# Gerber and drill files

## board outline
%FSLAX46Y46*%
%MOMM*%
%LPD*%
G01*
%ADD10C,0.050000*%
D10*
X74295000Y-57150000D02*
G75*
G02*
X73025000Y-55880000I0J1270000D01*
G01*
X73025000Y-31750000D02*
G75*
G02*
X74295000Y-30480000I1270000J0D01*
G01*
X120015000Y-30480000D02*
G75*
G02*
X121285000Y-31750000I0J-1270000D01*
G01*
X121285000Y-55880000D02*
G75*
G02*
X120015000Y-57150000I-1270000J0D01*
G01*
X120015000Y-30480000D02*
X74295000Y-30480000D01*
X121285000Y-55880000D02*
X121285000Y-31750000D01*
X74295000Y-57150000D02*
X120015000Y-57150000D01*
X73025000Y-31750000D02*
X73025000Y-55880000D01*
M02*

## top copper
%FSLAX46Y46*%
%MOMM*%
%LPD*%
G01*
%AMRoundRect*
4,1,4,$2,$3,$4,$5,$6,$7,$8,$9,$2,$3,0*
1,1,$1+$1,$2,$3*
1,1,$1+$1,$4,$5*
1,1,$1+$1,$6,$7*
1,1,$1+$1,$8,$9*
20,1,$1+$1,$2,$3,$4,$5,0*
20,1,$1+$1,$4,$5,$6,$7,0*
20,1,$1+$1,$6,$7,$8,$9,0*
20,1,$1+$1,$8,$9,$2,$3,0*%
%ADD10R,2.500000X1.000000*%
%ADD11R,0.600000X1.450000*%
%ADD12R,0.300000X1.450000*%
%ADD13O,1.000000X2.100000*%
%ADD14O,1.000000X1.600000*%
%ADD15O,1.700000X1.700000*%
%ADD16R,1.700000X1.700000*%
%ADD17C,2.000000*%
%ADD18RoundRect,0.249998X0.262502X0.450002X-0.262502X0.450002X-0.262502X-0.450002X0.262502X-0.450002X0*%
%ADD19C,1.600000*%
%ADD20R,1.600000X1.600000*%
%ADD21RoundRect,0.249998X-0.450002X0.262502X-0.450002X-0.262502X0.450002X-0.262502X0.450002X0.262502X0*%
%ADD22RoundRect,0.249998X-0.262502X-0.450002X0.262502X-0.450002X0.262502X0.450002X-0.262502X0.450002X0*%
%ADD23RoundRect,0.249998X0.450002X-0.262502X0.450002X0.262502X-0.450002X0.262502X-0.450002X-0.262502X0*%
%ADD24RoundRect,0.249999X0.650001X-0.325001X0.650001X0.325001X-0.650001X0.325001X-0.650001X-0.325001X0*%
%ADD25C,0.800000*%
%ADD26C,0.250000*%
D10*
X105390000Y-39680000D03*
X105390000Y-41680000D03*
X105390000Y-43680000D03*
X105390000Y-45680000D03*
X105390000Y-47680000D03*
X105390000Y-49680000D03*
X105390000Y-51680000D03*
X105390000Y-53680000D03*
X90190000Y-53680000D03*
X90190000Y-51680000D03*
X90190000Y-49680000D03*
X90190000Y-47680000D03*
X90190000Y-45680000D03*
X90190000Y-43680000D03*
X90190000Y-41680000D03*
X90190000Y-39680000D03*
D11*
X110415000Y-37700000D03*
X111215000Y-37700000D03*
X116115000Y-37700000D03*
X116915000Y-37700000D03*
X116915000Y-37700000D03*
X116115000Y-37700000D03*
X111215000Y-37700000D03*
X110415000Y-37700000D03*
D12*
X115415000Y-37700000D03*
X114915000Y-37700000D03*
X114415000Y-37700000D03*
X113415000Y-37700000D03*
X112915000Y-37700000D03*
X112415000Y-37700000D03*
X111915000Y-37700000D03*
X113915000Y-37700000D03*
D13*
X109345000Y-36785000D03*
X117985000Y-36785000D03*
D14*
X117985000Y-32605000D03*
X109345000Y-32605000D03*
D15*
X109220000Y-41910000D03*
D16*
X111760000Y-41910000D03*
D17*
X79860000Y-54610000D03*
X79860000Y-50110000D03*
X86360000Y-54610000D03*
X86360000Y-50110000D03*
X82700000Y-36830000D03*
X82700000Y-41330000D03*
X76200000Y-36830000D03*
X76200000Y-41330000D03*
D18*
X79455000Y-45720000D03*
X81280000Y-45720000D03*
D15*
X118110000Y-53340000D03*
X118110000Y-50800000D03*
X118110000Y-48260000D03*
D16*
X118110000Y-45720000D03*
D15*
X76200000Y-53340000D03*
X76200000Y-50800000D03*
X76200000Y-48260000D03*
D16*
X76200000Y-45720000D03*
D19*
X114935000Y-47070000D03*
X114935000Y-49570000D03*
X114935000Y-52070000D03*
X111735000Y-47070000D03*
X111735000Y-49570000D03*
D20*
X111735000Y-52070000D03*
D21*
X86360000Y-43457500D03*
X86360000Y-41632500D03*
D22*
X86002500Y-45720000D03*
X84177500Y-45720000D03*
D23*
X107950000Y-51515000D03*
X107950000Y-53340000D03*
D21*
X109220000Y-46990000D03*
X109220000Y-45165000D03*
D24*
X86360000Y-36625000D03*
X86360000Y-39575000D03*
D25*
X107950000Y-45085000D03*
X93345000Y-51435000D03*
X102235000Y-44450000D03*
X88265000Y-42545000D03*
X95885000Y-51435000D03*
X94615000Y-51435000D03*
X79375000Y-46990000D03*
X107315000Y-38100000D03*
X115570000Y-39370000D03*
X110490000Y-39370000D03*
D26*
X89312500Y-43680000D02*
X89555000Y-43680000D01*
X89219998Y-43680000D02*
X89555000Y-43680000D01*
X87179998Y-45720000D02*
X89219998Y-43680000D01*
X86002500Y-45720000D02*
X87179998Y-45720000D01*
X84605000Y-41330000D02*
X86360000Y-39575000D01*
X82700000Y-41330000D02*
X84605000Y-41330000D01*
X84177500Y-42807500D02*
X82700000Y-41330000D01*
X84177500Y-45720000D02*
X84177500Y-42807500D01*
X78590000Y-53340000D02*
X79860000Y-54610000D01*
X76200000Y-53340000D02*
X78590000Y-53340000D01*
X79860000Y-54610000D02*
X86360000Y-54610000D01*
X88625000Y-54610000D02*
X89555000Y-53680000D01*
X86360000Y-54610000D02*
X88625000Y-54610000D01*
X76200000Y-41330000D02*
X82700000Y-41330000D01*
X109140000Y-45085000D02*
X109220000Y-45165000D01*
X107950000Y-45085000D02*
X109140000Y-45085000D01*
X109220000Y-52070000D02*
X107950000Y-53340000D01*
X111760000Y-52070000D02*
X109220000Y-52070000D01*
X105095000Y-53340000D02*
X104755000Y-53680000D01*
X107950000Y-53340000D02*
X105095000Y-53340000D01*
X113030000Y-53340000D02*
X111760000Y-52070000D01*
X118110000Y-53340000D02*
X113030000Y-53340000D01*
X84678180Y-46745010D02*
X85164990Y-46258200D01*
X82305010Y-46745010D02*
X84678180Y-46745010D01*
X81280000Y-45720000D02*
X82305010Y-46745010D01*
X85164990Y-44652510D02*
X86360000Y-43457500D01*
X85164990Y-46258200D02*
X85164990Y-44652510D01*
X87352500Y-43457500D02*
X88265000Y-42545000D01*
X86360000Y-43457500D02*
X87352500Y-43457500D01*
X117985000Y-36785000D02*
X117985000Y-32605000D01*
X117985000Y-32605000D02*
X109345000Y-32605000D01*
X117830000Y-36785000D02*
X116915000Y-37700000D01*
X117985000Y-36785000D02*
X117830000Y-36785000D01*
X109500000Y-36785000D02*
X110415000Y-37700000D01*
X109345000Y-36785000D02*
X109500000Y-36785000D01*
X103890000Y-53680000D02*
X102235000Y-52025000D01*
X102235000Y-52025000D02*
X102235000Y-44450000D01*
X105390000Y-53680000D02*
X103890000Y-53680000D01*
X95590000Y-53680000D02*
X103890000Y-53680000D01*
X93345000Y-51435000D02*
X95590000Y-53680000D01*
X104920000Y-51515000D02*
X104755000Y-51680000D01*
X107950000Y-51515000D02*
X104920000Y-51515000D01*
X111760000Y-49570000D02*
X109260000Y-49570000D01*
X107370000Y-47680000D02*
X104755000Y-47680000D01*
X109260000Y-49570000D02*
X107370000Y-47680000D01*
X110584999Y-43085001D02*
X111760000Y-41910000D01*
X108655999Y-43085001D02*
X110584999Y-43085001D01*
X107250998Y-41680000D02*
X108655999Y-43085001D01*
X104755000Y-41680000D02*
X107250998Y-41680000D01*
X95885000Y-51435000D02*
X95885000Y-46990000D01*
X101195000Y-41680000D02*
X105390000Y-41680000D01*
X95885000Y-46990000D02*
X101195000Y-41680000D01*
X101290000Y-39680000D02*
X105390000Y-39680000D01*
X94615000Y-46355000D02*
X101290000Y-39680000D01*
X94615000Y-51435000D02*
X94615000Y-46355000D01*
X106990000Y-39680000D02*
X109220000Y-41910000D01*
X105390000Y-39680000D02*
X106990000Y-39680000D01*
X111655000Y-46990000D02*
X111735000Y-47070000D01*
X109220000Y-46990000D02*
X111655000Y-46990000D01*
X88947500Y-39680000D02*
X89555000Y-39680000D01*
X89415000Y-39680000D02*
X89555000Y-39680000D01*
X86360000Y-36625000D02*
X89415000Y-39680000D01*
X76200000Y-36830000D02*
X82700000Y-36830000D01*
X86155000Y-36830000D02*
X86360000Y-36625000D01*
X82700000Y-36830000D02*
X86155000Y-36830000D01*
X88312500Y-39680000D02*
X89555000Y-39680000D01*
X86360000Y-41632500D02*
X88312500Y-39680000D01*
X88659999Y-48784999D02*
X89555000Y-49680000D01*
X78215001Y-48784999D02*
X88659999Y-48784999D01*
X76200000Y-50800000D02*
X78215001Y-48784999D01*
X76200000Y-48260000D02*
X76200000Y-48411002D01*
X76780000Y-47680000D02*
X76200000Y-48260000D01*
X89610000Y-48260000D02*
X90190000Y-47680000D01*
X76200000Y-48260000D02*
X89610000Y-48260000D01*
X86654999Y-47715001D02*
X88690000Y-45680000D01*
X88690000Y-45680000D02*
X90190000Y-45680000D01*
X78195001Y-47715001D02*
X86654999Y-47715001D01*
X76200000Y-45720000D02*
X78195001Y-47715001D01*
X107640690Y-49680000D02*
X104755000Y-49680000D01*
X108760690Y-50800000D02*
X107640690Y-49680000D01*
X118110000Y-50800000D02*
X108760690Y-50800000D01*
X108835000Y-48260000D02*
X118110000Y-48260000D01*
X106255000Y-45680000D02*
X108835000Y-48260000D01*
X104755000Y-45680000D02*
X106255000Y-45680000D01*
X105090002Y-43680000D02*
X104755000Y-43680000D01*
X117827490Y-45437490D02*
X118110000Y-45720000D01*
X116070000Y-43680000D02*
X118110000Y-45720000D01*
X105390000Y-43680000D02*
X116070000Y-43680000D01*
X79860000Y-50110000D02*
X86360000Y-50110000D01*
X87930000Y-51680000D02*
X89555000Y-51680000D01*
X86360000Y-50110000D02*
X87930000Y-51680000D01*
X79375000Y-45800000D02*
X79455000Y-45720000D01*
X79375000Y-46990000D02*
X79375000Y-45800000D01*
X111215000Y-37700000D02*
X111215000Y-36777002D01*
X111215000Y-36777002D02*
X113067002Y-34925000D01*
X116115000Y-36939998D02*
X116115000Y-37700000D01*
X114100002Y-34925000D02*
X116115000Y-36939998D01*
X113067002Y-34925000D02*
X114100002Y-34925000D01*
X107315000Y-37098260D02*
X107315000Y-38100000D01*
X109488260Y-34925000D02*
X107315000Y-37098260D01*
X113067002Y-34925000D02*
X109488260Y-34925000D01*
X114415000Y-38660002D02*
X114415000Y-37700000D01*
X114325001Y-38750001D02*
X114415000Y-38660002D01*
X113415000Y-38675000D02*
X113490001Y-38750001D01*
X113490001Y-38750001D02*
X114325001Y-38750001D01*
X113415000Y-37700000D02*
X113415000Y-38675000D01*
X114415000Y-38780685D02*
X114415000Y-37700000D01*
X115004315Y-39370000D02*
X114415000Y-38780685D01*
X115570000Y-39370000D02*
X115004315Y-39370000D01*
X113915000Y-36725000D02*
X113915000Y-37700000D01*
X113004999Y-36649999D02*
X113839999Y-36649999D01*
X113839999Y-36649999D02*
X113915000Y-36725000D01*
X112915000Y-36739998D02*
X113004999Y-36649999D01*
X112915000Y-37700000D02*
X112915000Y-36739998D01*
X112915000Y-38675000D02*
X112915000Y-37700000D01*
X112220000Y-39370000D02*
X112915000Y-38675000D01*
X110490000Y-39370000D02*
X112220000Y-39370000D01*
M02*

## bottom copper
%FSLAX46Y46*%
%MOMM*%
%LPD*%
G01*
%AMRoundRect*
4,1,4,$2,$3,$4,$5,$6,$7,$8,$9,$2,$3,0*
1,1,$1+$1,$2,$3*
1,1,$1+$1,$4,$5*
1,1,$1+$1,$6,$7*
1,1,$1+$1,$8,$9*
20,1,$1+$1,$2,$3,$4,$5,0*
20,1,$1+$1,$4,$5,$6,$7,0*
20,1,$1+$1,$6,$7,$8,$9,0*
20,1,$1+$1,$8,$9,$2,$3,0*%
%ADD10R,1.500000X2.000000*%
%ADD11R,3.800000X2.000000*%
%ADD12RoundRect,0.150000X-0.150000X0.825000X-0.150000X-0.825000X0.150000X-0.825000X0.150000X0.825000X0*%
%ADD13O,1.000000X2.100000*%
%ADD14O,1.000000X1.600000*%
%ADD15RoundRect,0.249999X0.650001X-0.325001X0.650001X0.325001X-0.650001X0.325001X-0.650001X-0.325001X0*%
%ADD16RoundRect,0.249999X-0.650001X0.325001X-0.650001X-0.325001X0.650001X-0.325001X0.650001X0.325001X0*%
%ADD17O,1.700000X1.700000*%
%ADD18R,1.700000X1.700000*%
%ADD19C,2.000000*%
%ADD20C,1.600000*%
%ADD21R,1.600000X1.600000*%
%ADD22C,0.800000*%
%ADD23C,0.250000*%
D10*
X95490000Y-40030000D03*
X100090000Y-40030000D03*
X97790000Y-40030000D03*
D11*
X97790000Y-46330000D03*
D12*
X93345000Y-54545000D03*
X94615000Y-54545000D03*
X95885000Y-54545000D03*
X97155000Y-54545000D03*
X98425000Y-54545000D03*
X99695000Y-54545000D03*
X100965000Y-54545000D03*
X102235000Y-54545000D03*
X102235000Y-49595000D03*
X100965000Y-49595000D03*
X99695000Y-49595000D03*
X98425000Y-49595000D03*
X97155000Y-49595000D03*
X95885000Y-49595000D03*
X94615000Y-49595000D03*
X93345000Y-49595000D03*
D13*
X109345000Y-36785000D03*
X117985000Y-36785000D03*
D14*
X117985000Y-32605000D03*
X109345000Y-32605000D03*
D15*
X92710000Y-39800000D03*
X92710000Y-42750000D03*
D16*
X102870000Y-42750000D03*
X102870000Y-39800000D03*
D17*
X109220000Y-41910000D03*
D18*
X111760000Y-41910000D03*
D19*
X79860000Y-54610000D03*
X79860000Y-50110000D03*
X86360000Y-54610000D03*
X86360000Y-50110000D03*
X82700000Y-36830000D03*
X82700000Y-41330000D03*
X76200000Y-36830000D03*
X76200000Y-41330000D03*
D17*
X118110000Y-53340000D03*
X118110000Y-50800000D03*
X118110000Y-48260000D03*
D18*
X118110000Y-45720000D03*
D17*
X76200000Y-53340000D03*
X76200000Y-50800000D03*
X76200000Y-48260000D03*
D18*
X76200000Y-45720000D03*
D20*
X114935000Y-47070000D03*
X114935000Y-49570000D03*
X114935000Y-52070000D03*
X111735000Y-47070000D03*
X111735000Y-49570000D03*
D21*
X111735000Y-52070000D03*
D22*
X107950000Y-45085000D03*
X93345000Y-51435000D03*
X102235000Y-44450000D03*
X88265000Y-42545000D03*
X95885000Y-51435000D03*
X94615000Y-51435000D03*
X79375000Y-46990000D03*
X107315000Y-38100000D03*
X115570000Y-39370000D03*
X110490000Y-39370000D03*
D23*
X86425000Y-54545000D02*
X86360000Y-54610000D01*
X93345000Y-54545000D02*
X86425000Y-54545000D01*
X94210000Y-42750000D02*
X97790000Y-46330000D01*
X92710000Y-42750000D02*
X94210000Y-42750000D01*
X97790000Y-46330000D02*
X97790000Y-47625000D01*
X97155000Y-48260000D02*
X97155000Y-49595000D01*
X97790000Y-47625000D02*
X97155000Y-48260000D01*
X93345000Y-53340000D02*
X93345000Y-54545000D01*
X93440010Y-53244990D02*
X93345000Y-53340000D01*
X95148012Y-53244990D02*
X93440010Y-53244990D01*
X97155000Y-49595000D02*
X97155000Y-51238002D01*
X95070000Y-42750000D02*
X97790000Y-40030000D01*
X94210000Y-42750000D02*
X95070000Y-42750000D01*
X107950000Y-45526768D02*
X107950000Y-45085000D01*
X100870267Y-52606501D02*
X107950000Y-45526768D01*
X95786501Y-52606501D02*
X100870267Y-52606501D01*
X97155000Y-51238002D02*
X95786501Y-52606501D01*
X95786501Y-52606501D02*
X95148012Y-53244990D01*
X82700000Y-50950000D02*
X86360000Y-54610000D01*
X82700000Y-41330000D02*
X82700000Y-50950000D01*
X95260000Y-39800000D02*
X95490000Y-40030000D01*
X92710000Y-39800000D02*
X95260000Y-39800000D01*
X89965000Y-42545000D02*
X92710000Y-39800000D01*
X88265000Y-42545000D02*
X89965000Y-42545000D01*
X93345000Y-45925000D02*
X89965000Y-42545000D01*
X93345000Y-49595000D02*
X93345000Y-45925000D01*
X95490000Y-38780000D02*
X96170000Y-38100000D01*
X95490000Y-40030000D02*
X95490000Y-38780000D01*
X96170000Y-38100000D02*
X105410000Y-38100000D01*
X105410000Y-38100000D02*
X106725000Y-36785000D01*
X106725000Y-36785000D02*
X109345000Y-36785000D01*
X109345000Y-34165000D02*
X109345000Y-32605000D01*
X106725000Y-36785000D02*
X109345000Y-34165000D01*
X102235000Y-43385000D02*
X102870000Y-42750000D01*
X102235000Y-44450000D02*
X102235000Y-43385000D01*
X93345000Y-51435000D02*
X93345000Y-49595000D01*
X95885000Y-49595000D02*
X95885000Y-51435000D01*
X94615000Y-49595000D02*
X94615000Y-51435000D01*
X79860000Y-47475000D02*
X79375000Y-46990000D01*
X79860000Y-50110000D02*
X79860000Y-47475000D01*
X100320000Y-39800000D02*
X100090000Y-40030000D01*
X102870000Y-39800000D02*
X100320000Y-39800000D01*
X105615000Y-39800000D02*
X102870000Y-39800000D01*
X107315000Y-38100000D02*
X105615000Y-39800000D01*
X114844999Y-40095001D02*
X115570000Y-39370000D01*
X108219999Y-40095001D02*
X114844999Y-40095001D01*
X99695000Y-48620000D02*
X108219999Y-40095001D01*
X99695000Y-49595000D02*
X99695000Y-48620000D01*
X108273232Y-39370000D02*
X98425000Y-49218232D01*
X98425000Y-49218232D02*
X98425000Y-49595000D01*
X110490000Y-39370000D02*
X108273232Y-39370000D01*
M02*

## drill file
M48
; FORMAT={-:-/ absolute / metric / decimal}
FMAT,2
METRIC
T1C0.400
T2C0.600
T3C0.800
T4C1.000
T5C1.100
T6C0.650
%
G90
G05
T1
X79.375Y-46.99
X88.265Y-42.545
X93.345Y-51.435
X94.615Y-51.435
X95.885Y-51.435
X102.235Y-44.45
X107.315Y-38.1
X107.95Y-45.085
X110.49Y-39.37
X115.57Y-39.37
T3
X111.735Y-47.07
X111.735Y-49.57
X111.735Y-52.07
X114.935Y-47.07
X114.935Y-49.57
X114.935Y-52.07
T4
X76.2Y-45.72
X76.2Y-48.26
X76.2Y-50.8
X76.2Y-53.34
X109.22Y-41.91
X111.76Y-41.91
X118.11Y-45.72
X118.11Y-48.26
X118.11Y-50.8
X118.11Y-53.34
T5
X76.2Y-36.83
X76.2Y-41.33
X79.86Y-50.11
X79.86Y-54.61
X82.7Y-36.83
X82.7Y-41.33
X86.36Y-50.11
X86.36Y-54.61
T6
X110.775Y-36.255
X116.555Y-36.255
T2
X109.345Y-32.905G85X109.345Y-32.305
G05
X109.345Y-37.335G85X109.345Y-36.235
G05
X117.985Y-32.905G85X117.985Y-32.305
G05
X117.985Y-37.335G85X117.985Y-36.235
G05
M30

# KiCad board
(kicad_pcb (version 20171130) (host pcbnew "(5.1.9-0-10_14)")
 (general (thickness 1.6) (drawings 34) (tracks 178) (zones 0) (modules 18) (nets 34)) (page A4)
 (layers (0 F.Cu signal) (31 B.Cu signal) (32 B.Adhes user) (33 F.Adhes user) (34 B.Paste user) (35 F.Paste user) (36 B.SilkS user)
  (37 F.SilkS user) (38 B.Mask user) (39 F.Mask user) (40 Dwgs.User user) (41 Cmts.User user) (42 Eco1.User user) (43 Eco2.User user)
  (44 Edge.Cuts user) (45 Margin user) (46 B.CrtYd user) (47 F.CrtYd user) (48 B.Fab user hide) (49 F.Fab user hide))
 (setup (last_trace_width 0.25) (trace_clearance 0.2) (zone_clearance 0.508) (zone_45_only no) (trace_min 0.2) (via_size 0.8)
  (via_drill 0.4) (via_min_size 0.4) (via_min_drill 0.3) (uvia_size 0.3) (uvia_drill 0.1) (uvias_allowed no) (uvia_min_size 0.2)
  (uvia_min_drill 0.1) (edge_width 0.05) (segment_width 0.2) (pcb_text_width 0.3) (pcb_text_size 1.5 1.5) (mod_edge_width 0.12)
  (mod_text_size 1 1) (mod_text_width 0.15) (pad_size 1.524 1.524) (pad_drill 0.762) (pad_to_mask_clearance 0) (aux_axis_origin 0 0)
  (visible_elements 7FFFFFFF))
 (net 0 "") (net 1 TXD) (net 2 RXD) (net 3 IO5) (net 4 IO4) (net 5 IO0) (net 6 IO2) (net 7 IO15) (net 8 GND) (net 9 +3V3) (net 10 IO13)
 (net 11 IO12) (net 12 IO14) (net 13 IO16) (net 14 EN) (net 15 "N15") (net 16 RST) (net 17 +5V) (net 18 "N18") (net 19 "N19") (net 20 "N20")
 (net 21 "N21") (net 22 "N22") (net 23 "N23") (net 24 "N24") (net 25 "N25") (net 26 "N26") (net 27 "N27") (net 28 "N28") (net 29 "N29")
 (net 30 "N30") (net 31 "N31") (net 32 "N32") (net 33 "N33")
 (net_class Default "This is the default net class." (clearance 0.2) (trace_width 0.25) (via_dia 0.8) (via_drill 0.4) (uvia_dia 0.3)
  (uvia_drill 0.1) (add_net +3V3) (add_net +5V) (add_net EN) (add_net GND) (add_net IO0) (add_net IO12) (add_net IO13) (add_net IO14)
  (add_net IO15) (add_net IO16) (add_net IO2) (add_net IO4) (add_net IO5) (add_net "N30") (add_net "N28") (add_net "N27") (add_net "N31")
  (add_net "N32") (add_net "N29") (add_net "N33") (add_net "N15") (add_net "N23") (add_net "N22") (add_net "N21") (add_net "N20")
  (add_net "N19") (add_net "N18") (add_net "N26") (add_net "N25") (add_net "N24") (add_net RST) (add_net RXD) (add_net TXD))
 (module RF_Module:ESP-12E (layer F.Cu) (at 97.79 43.18)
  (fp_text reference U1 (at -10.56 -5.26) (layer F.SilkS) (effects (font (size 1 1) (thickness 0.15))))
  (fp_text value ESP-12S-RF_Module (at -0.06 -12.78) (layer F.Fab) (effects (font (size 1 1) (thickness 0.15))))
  (pad 16 smd rect (at 7.6 -3.5) (size 2.5 1) (layers F.Cu F.Paste F.Mask) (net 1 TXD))
  (pad 15 smd rect (at 7.6 -1.5) (size 2.5 1) (layers F.Cu F.Paste F.Mask) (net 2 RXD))
  (pad 14 smd rect (at 7.6 0.5) (size 2.5 1) (layers F.Cu F.Paste F.Mask) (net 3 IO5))
  (pad 13 smd rect (at 7.6 2.5) (size 2.5 1) (layers F.Cu F.Paste F.Mask) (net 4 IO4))
  (pad 12 smd rect (at 7.6 4.5) (size 2.5 1) (layers F.Cu F.Paste F.Mask) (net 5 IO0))
  (pad 11 smd rect (at 7.6 6.5) (size 2.5 1) (layers F.Cu F.Paste F.Mask) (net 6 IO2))
  (pad 10 smd rect (at 7.6 8.5) (size 2.5 1) (layers F.Cu F.Paste F.Mask) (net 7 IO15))
  (pad 9 smd rect (at 7.6 10.5) (size 2.5 1) (layers F.Cu F.Paste F.Mask) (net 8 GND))
  (pad 8 smd rect (at -7.6 10.5) (size 2.5 1) (layers F.Cu F.Paste F.Mask) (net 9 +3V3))
  (pad 7 smd rect (at -7.6 8.5) (size 2.5 1) (layers F.Cu F.Paste F.Mask) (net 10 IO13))
  (pad 6 smd rect (at -7.6 6.5) (size 2.5 1) (layers F.Cu F.Paste F.Mask) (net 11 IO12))
  (pad 5 smd rect (at -7.6 4.5) (size 2.5 1) (layers F.Cu F.Paste F.Mask) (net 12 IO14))
  (pad 4 smd rect (at -7.6 2.5) (size 2.5 1) (layers F.Cu F.Paste F.Mask) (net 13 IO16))
  (pad 3 smd rect (at -7.6 0.5) (size 2.5 1) (layers F.Cu F.Paste F.Mask) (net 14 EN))
  (pad 2 smd rect (at -7.6 -1.5) (size 2.5 1) (layers F.Cu F.Paste F.Mask) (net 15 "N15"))
  (pad 1 smd rect (at -7.6 -3.5) (size 2.5 1) (layers F.Cu F.Paste F.Mask) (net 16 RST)))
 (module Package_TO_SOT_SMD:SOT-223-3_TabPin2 (layer B.Cu) (at 97.79 43.18 270)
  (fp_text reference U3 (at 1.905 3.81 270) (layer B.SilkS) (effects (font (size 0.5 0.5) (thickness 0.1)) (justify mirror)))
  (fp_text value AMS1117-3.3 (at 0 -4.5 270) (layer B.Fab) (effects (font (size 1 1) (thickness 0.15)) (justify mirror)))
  (pad 1 smd rect (at -3.15 2.3 270) (size 2 1.5) (layers B.Cu B.Paste B.Mask) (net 8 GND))
  (pad 3 smd rect (at -3.15 -2.3 270) (size 2 1.5) (layers B.Cu B.Paste B.Mask) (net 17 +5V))
  (pad 2 smd rect (at -3.15 0 270) (size 2 1.5) (layers B.Cu B.Paste B.Mask) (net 9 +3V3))
  (pad 2 smd rect (at 3.15 0 270) (size 2 3.8) (layers B.Cu B.Paste B.Mask) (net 9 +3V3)))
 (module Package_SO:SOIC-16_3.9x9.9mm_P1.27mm (layer B.Cu) (at 97.79 52.07 270)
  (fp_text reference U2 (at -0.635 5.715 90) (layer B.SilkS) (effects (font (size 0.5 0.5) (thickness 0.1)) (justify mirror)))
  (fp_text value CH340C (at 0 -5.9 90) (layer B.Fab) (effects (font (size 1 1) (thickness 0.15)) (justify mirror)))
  (pad 16 smd roundrect (at 2.475 4.445 270) (size 1.95 0.6) (layers B.Cu B.Paste B.Mask) (roundrect_rratio 0.25) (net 9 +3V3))
  (pad 15 smd roundrect (at 2.475 3.175 270) (size 1.95 0.6) (layers B.Cu B.Paste B.Mask) (roundrect_rratio 0.25) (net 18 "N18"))
  (pad 14 smd roundrect (at 2.475 1.905 270) (size 1.95 0.6) (layers B.Cu B.Paste B.Mask) (roundrect_rratio 0.25) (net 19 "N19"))
  (pad 13 smd roundrect (at 2.475 0.635 270) (size 1.95 0.6) (layers B.Cu B.Paste B.Mask) (roundrect_rratio 0.25) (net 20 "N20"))
  (pad 12 smd roundrect (at 2.475 -0.635 270) (size 1.95 0.6) (layers B.Cu B.Paste B.Mask) (roundrect_rratio 0.25) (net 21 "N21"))
  (pad 11 smd roundrect (at 2.475 -1.905 270) (size 1.95 0.6) (layers B.Cu B.Paste B.Mask) (roundrect_rratio 0.25) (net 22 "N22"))
  (pad 10 smd roundrect (at 2.475 -3.175 270) (size 1.95 0.6) (layers B.Cu B.Paste B.Mask) (roundrect_rratio 0.25) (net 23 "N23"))
  (pad 9 smd roundrect (at 2.475 -4.445 270) (size 1.95 0.6) (layers B.Cu B.Paste B.Mask) (roundrect_rratio 0.25) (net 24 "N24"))
  (pad 8 smd roundrect (at -2.475 -4.445 270) (size 1.95 0.6) (layers B.Cu B.Paste B.Mask) (roundrect_rratio 0.25) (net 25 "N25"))
  (pad 7 smd roundrect (at -2.475 -3.175 270) (size 1.95 0.6) (layers B.Cu B.Paste B.Mask) (roundrect_rratio 0.25) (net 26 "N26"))
  (pad 6 smd roundrect (at -2.475 -1.905 270) (size 1.95 0.6) (layers B.Cu B.Paste B.Mask) (roundrect_rratio 0.25) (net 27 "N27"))
  (pad 5 smd roundrect (at -2.475 -0.635 270) (size 1.95 0.6) (layers B.Cu B.Paste B.Mask) (roundrect_rratio 0.25) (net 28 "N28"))
  (pad 4 smd roundrect (at -2.475 0.635 270) (size 1.95 0.6) (layers B.Cu B.Paste B.Mask) (roundrect_rratio 0.25) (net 9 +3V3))
  (pad 3 smd roundrect (at -2.475 1.905 270) (size 1.95 0.6) (layers B.Cu B.Paste B.Mask) (roundrect_rratio 0.25) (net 2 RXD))
  (pad 2 smd roundrect (at -2.475 3.175 270) (size 1.95 0.6) (layers B.Cu B.Paste B.Mask) (roundrect_rratio 0.25) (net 1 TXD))
  (pad 1 smd roundrect (at -2.475 4.445 270) (size 1.95 0.6) (layers B.Cu B.Paste B.Mask) (roundrect_rratio 0.25) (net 8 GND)))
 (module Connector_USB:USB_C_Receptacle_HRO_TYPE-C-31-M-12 (layer F.Cu) (at 113.665 33.655 180)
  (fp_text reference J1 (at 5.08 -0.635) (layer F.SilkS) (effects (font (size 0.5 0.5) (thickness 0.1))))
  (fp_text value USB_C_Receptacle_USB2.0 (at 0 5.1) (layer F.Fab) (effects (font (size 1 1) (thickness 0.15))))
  (pad B1 smd rect (at 3.25 -4.045 180) (size 0.6 1.45) (layers F.Cu F.Paste F.Mask) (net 8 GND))
  (pad A9 smd rect (at 2.45 -4.045 180) (size 0.6 1.45) (layers F.Cu F.Paste F.Mask) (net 17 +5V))
  (pad B9 smd rect (at -2.45 -4.045 180) (size 0.6 1.45) (layers F.Cu F.Paste F.Mask) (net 17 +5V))
  (pad B12 smd rect (at -3.25 -4.045 180) (size 0.6 1.45) (layers F.Cu F.Paste F.Mask) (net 8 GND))
  (pad A1 smd rect (at -3.25 -4.045 180) (size 0.6 1.45) (layers F.Cu F.Paste F.Mask) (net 8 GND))
  (pad A4 smd rect (at -2.45 -4.045 180) (size 0.6 1.45) (layers F.Cu F.Paste F.Mask) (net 17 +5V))
  (pad B4 smd rect (at 2.45 -4.045 180) (size 0.6 1.45) (layers F.Cu F.Paste F.Mask) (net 17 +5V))
  (pad A12 smd rect (at 3.25 -4.045 180) (size 0.6 1.45) (layers F.Cu F.Paste F.Mask) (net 8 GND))
  (pad B8 smd rect (at -1.75 -4.045 180) (size 0.3 1.45) (layers F.Cu F.Paste F.Mask) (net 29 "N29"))
  (pad A5 smd rect (at -1.25 -4.045 180) (size 0.3 1.45) (layers F.Cu F.Paste F.Mask) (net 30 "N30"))
  (pad B7 smd rect (at -0.75 -4.045 180) (size 0.3 1.45) (layers F.Cu F.Paste F.Mask) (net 27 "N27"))
  (pad A7 smd rect (at 0.25 -4.045 180) (size 0.3 1.45) (layers F.Cu F.Paste F.Mask) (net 27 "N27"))
  (pad B6 smd rect (at 0.75 -4.045 180) (size 0.3 1.45) (layers F.Cu F.Paste F.Mask) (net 28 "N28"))
  (pad A8 smd rect (at 1.25 -4.045 180) (size 0.3 1.45) (layers F.Cu F.Paste F.Mask) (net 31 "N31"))
  (pad B5 smd rect (at 1.75 -4.045 180) (size 0.3 1.45) (layers F.Cu F.Paste F.Mask) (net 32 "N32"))
  (pad A6 smd rect (at -0.25 -4.045 180) (size 0.3 1.45) (layers F.Cu F.Paste F.Mask) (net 28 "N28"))
  (pad S1 thru_hole oval (at 4.32 -3.13 180) (size 1 2.1) (drill oval 0.6 1.7) (layers *.Cu *.Mask) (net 8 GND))
  (pad S1 thru_hole oval (at -4.32 -3.13 180) (size 1 2.1) (drill oval 0.6 1.7) (layers *.Cu *.Mask) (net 8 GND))
  (pad "" np_thru_hole circle (at -2.89 -2.6 180) (size 0.65 0.65) (drill 0.65) (layers *.Cu *.Mask))
  (pad S1 thru_hole oval (at -4.32 1.05 180) (size 1 1.6) (drill oval 0.6 1.2) (layers *.Cu *.Mask) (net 8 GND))
  (pad "" np_thru_hole circle (at 2.89 -2.6 180) (size 0.65 0.65) (drill 0.65) (layers *.Cu *.Mask))
  (pad S1 thru_hole oval (at 4.32 1.05 180) (size 1 1.6) (drill oval 0.6 1.2) (layers *.Cu *.Mask) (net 8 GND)))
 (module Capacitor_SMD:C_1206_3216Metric (layer B.Cu) (at 92.71 41.275 90)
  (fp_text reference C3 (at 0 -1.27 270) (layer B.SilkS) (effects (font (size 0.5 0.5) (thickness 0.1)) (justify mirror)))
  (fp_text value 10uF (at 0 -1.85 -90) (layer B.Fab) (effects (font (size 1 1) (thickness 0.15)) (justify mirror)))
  (pad 2 smd roundrect (at 1.475 0 90) (size 1.15 1.8) (layers B.Cu B.Paste B.Mask) (roundrect_rratio 0.2173904347826087) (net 8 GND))
  (pad 1 smd roundrect (at -1.475 0 90) (size 1.15 1.8) (layers B.Cu B.Paste B.Mask) (roundrect_rratio 0.2173904347826087) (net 9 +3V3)))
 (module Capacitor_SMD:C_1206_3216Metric (layer B.Cu) (at 102.87 41.275 270)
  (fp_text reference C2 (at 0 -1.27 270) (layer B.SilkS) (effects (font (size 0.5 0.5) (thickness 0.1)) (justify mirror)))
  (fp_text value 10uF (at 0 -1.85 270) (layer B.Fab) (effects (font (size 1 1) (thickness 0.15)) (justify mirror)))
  (pad 2 smd roundrect (at 1.475 0 270) (size 1.15 1.8) (layers B.Cu B.Paste B.Mask) (roundrect_rratio 0.2173904347826087) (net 8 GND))
  (pad 1 smd roundrect (at -1.475 0 270) (size 1.15 1.8) (layers B.Cu B.Paste B.Mask) (roundrect_rratio 0.2173904347826087) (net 17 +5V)))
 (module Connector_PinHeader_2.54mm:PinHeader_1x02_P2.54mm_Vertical (layer B.Cu) (at 111.76 41.91 90)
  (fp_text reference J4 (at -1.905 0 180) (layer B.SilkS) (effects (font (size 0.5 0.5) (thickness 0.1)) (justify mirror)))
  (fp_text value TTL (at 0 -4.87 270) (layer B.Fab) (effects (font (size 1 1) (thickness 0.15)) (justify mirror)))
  (pad 2 thru_hole oval (at 0 -2.54 90) (size 1.7 1.7) (drill 1) (layers *.Cu *.Mask) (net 1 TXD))
  (pad 1 thru_hole rect (at 0 0 90) (size 1.7 1.7) (drill 1) (layers *.Cu *.Mask) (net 2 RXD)))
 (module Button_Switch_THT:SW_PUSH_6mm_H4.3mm (layer F.Cu) (at 86.36 54.61 180)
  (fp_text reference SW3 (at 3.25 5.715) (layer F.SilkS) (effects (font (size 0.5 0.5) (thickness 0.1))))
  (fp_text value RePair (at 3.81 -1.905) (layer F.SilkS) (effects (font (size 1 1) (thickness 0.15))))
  (pad 1 thru_hole circle (at 6.5 0 270) (size 2 2) (drill 1.1) (layers *.Cu *.Mask) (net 9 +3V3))
  (pad 2 thru_hole circle (at 6.5 4.5 270) (size 2 2) (drill 1.1) (layers *.Cu *.Mask) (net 10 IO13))
  (pad 1 thru_hole circle (at 0 0 270) (size 2 2) (drill 1.1) (layers *.Cu *.Mask) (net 9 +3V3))
  (pad 2 thru_hole circle (at 0 4.5 270) (size 2 2) (drill 1.1) (layers *.Cu *.Mask) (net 10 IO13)))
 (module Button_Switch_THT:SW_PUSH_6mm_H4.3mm (layer F.Cu) (at 76.2 36.83)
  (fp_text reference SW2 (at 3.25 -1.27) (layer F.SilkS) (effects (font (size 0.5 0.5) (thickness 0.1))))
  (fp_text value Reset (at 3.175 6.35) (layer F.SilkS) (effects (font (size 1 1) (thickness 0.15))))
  (pad 1 thru_hole circle (at 6.5 0 90) (size 2 2) (drill 1.1) (layers *.Cu *.Mask) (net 16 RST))
  (pad 2 thru_hole circle (at 6.5 4.5 90) (size 2 2) (drill 1.1) (layers *.Cu *.Mask) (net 9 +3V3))
  (pad 1 thru_hole circle (at 0 0 90) (size 2 2) (drill 1.1) (layers *.Cu *.Mask) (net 16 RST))
  (pad 2 thru_hole circle (at 0 4.5 90) (size 2 2) (drill 1.1) (layers *.Cu *.Mask) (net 9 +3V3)))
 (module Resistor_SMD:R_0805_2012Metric (layer F.Cu) (at 80.3675 45.72 180)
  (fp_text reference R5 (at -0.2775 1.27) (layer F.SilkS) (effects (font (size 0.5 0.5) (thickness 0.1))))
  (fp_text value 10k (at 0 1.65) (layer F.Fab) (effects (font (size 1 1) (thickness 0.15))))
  (pad 2 smd roundrect (at 0.9125 0 180) (size 1.025 1.4) (layers F.Cu F.Paste F.Mask) (roundrect_rratio 0.2439004878048781) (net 10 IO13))
  (pad 1 smd roundrect (at -0.9125 0 180) (size 1.025 1.4) (layers F.Cu F.Paste F.Mask) (roundrect_rratio 0.2439004878048781) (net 8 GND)))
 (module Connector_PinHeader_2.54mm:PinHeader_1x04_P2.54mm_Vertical (layer B.Cu) (at 118.11 45.72 180)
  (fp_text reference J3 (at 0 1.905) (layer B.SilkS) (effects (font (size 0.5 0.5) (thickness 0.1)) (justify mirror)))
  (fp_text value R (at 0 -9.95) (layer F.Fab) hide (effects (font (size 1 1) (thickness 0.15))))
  (pad 4 thru_hole oval (at 0 -7.62 180) (size 1.7 1.7) (drill 1) (layers *.Cu *.Mask) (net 8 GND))
  (pad 3 thru_hole oval (at 0 -5.08 180) (size 1.7 1.7) (drill 1) (layers *.Cu *.Mask) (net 6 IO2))
  (pad 2 thru_hole oval (at 0 -2.54 180) (size 1.7 1.7) (drill 1) (layers *.Cu *.Mask) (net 4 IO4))
  (pad 1 thru_hole rect (at 0 0 180) (size 1.7 1.7) (drill 1) (layers *.Cu *.Mask) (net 3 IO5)))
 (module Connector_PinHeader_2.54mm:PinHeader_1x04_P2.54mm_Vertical (layer B.Cu) (at 76.2 45.72 180)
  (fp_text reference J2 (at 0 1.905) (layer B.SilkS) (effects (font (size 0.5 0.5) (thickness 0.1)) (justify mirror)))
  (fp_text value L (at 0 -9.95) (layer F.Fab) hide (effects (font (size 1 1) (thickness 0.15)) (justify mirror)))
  (pad 4 thru_hole oval (at 0 -7.62 180) (size 1.7 1.7) (drill 1) (layers *.Cu *.Mask) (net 9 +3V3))
  (pad 3 thru_hole oval (at 0 -5.08 180) (size 1.7 1.7) (drill 1) (layers *.Cu *.Mask) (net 11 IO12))
  (pad 2 thru_hole oval (at 0 -2.54 180) (size 1.7 1.7) (drill 1) (layers *.Cu *.Mask) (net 12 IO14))
  (pad 1 thru_hole rect (at 0 0 180) (size 1.7 1.7) (drill 1) (layers *.Cu *.Mask) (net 13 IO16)))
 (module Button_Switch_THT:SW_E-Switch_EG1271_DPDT (layer F.Cu) (at 111.735 52.07 90)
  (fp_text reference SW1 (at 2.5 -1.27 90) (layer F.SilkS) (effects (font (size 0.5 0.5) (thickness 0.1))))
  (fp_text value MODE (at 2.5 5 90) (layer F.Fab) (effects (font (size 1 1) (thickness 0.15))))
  (pad 6 thru_hole circle (at 5 3.2 90) (size 1.6 1.6) (drill 0.8) (layers *.Cu *.Mask))
  (pad 5 thru_hole circle (at 2.5 3.2 90) (size 1.6 1.6) (drill 0.8) (layers *.Cu *.Mask))
  (pad 4 thru_hole circle (at 0 3.2 90) (size 1.6 1.6) (drill 0.8) (layers *.Cu *.Mask))
  (pad 3 thru_hole circle (at 5 0 90) (size 1.6 1.6) (drill 0.8) (layers *.Cu *.Mask) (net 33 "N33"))
  (pad 2 thru_hole circle (at 2.5 0 90) (size 1.6 1.6) (drill 0.8) (layers *.Cu *.Mask) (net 5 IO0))
  (pad 1 thru_hole rect (at 0 0 90) (size 1.6 1.6) (drill 0.8) (layers *.Cu *.Mask) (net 8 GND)))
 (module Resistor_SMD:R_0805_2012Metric (layer F.Cu) (at 86.36 42.545 270)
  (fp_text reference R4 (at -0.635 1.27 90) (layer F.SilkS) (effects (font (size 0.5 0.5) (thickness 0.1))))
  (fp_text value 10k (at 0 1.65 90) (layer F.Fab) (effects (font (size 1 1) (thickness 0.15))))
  (pad 2 smd roundrect (at 0.9125 0 270) (size 1.025 1.4) (layers F.Cu F.Paste F.Mask) (roundrect_rratio 0.2439004878048781) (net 8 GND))
  (pad 1 smd roundrect (at -0.9125 0 270) (size 1.025 1.4) (layers F.Cu F.Paste F.Mask) (roundrect_rratio 0.2439004878048781) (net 16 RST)))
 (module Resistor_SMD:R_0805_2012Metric (layer F.Cu) (at 85.09 45.72)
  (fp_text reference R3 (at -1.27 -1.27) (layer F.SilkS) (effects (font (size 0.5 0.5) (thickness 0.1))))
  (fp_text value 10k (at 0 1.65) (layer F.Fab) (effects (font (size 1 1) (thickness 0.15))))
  (pad 2 smd roundrect (at 0.9125 0) (size 1.025 1.4) (layers F.Cu F.Paste F.Mask) (roundrect_rratio 0.2439004878048781) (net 14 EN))
  (pad 1 smd roundrect (at -0.9125 0) (size 1.025 1.4) (layers F.Cu F.Paste F.Mask) (roundrect_rratio 0.2439004878048781) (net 9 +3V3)))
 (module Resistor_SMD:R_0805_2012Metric (layer F.Cu) (at 107.95 52.4275 90)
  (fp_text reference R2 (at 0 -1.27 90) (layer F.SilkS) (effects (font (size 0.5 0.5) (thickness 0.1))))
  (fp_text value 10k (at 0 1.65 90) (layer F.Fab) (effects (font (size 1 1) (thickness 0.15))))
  (pad 2 smd roundrect (at 0.9125 0 90) (size 1.025 1.4) (layers F.Cu F.Paste F.Mask) (roundrect_rratio 0.2439004878048781) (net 7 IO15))
  (pad 1 smd roundrect (at -0.9125 0 90) (size 1.025 1.4) (layers F.Cu F.Paste F.Mask) (roundrect_rratio 0.2439004878048781) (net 8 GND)))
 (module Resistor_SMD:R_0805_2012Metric (layer F.Cu) (at 109.22 46.0775 270)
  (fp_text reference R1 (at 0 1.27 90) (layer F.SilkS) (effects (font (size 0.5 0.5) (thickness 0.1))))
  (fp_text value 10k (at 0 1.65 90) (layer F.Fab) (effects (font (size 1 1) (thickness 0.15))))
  (pad 2 smd roundrect (at 0.9125 0 270) (size 1.025 1.4) (layers F.Cu F.Paste F.Mask) (roundrect_rratio 0.2439004878048781) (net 33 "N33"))
  (pad 1 smd roundrect (at -0.9125 0 270) (size 1.025 1.4) (layers F.Cu F.Paste F.Mask) (roundrect_rratio 0.2439004878048781) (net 9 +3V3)))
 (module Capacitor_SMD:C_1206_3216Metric (layer F.Cu) (at 86.36 38.1 90)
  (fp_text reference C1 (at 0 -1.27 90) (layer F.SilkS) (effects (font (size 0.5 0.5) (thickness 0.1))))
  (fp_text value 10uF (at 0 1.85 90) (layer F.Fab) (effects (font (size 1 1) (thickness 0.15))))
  (pad 2 smd roundrect (at 1.475 0 90) (size 1.15 1.8) (layers F.Cu F.Paste F.Mask) (roundrect_rratio 0.2173904347826087) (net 16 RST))
  (pad 1 smd roundrect (at -1.475 0 90) (size 1.15 1.8) (layers F.Cu F.Paste F.Mask) (roundrect_rratio 0.2173904347826087) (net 9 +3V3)))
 (gr_arc (start 74.295 55.88) (end 73.025 55.88) (angle -90) (layer Edge.Cuts) (width 0.05))
 (gr_arc (start 74.295 31.75) (end 74.295 30.48) (angle -90) (layer Edge.Cuts) (width 0.05))
 (gr_arc (start 120.015 31.75) (end 121.285 31.75) (angle -90) (layer Edge.Cuts) (width 0.05))
 (gr_arc (start 120.015 55.88) (end 120.015 57.15) (angle -90) (layer Edge.Cuts) (width 0.05))
 (gr_line (start 120.015 30.48) (end 74.295 30.48) (layer Edge.Cuts) (width 0.05))
 (gr_line (start 121.285 55.88) (end 121.285 31.75) (layer Edge.Cuts) (width 0.05))
 (gr_line (start 74.295 57.15) (end 120.015 57.15) (layer Edge.Cuts) (width 0.05))
 (gr_line (start 73.025 31.75) (end 73.025 55.88) (layer Edge.Cuts) (width 0.05))
 (segment (start 89.3125 43.68) (end 89.555 43.68) (width 0.25) (layer F.Cu) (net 14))
 (segment (start 89.219998 43.68) (end 89.555 43.68) (width 0.25) (layer F.Cu) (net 14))
 (segment (start 87.179998 45.72) (end 89.219998 43.68) (width 0.25) (layer F.Cu) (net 14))
 (segment (start 86.0025 45.72) (end 87.179998 45.72) (width 0.25) (layer F.Cu) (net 14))
 (via (at 107.95 45.085) (size 0.8) (drill 0.4) (layers F.Cu B.Cu) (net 9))
 (segment (start 84.605 41.33) (end 86.36 39.575) (width 0.25) (layer F.Cu) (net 9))
 (segment (start 82.7 41.33) (end 84.605 41.33) (width 0.25) (layer F.Cu) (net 9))
 (segment (start 84.1775 42.8075) (end 82.7 41.33) (width 0.25) (layer F.Cu) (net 9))
 (segment (start 84.1775 45.72) (end 84.1775 42.8075) (width 0.25) (layer F.Cu) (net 9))
 (segment (start 78.59 53.34) (end 79.86 54.61) (width 0.25) (layer F.Cu) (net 9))
 (segment (start 76.2 53.34) (end 78.59 53.34) (width 0.25) (layer F.Cu) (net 9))
 (segment (start 79.86 54.61) (end 86.36 54.61) (width 0.25) (layer F.Cu) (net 9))
 (segment (start 88.625 54.61) (end 89.555 53.68) (width 0.25) (layer F.Cu) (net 9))
 (segment (start 86.36 54.61) (end 88.625 54.61) (width 0.25) (layer F.Cu) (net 9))
 (segment (start 86.425 54.545) (end 86.36 54.61) (width 0.25) (layer B.Cu) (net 9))
 (segment (start 93.345 54.545) (end 86.425 54.545) (width 0.25) (layer B.Cu) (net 9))
 (segment (start 94.21 42.75) (end 97.79 46.33) (width 0.25) (layer B.Cu) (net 9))
 (segment (start 92.71 42.75) (end 94.21 42.75) (width 0.25) (layer B.Cu) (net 9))
 (segment (start 97.79 46.33) (end 97.79 47.625) (width 0.25) (layer B.Cu) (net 9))
 (segment (start 97.155 48.26) (end 97.155 49.595) (width 0.25) (layer B.Cu) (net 9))
 (segment (start 97.79 47.625) (end 97.155 48.26) (width 0.25) (layer B.Cu) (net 9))
 (segment (start 93.345 53.34) (end 93.345 54.545) (width 0.25) (layer B.Cu) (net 9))
 (segment (start 93.44001 53.24499) (end 93.345 53.34) (width 0.25) (layer B.Cu) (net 9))
 (segment (start 95.148012 53.24499) (end 93.44001 53.24499) (width 0.25) (layer B.Cu) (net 9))
 (segment (start 97.155 49.595) (end 97.155 51.238002) (width 0.25) (layer B.Cu) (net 9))
 (segment (start 95.07 42.75) (end 97.79 40.03) (width 0.25) (layer B.Cu) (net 9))
 (segment (start 94.21 42.75) (end 95.07 42.75) (width 0.25) (layer B.Cu) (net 9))
 (segment (start 76.2 41.33) (end 82.7 41.33) (width 0.25) (layer F.Cu) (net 9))
 (segment (start 107.95 45.526768) (end 107.95 45.085) (width 0.25) (layer B.Cu) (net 9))
 (segment (start 100.870267 52.606501) (end 107.95 45.526768) (width 0.25) (layer B.Cu) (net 9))
 (segment (start 95.786501 52.606501) (end 100.870267 52.606501) (width 0.25) (layer B.Cu) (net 9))
 (segment (start 97.155 51.238002) (end 95.786501 52.606501) (width 0.25) (layer B.Cu) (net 9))
 (segment (start 95.786501 52.606501) (end 95.148012 53.24499) (width 0.25) (layer B.Cu) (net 9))
 (segment (start 109.14 45.085) (end 109.22 45.165) (width 0.25) (layer F.Cu) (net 9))
 (segment (start 107.95 45.085) (end 109.14 45.085) (width 0.25) (layer F.Cu) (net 9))
 (segment (start 82.7 50.95) (end 86.36 54.61) (width 0.25) (layer B.Cu) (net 9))
 (segment (start 82.7 41.33) (end 82.7 50.95) (width 0.25) (layer B.Cu) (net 9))
 (via (at 93.345 51.435) (size 0.8) (drill 0.4) (layers F.Cu B.Cu) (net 8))
 (via (at 102.235 44.45) (size 0.8) (drill 0.4) (layers F.Cu B.Cu) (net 8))
 (via (at 88.265 42.545) (size 0.8) (drill 0.4) (layers F.Cu B.Cu) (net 8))
 (segment (start 109.22 52.07) (end 107.95 53.34) (width 0.25) (layer F.Cu) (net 8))
 (segment (start 111.76 52.07) (end 109.22 52.07) (width 0.25) (layer F.Cu) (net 8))
 (segment (start 105.095 53.34) (end 104.755 53.68) (width 0.25) (layer F.Cu) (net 8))
 (segment (start 107.95 53.34) (end 105.095 53.34) (width 0.25) (layer F.Cu) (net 8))
 (segment (start 113.03 53.34) (end 111.76 52.07) (width 0.25) (layer F.Cu) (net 8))
 (segment (start 118.11 53.34) (end 113.03 53.34) (width 0.25) (layer F.Cu) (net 8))
 (segment (start 84.67818 46.74501) (end 85.16499 46.2582) (width 0.25) (layer F.Cu) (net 8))
 (segment (start 82.30501 46.74501) (end 84.67818 46.74501) (width 0.25) (layer F.Cu) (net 8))
 (segment (start 81.28 45.72) (end 82.30501 46.74501) (width 0.25) (layer F.Cu) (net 8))
 (segment (start 85.16499 44.65251) (end 86.36 43.4575) (width 0.25) (layer F.Cu) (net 8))
 (segment (start 85.16499 46.2582) (end 85.16499 44.65251) (width 0.25) (layer F.Cu) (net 8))
 (segment (start 95.26 39.8) (end 95.49 40.03) (width 0.25) (layer B.Cu) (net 8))
 (segment (start 92.71 39.8) (end 95.26 39.8) (width 0.25) (layer B.Cu) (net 8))
 (segment (start 87.3525 43.4575) (end 88.265 42.545) (width 0.25) (layer F.Cu) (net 8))
 (segment (start 86.36 43.4575) (end 87.3525 43.4575) (width 0.25) (layer F.Cu) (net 8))
 (segment (start 89.965 42.545) (end 92.71 39.8) (width 0.25) (layer B.Cu) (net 8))
 (segment (start 88.265 42.545) (end 89.965 42.545) (width 0.25) (layer B.Cu) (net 8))
 (segment (start 93.345 45.925) (end 89.965 42.545) (width 0.25) (layer B.Cu) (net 8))
 (segment (start 93.345 49.595) (end 93.345 45.925) (width 0.25) (layer B.Cu) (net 8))
 (segment (start 117.985 36.785) (end 117.985 32.605) (width 0.25) (layer F.Cu) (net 8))
 (segment (start 117.985 32.605) (end 109.345 32.605) (width 0.25) (layer F.Cu) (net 8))
 (segment (start 117.83 36.785) (end 116.915 37.7) (width 0.25) (layer F.Cu) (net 8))
 (segment (start 117.985 36.785) (end 117.83 36.785) (width 0.25) (layer F.Cu) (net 8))
 (segment (start 109.5 36.785) (end 110.415 37.7) (width 0.25) (layer F.Cu) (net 8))
 (segment (start 109.345 36.785) (end 109.5 36.785) (width 0.25) (layer F.Cu) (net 8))
 (segment (start 95.49 38.78) (end 96.17 38.1) (width 0.25) (layer B.Cu) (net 8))
 (segment (start 95.49 40.03) (end 95.49 38.78) (width 0.25) (layer B.Cu) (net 8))
 (segment (start 96.17 38.1) (end 105.41 38.1) (width 0.25) (layer B.Cu) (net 8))
 (segment (start 105.41 38.1) (end 106.725 36.785) (width 0.25) (layer B.Cu) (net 8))
 (segment (start 103.89 53.68) (end 102.235 52.025) (width 0.25) (layer F.Cu) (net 8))
 (segment (start 102.235 52.025) (end 102.235 44.45) (width 0.25) (layer F.Cu) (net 8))
 (segment (start 105.39 53.68) (end 103.89 53.68) (width 0.25) (layer F.Cu) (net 8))
 (segment (start 106.725 36.785) (end 109.345 36.785) (width 0.25) (layer B.Cu) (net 8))
 (segment (start 109.345 34.165) (end 109.345 32.605) (width 0.25) (layer B.Cu) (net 8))
 (segment (start 106.725 36.785) (end 109.345 34.165) (width 0.25) (layer B.Cu) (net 8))
 (segment (start 102.235 43.385) (end 102.87 42.75) (width 0.25) (layer B.Cu) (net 8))
 (segment (start 102.235 44.45) (end 102.235 43.385) (width 0.25) (layer B.Cu) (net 8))
 (segment (start 93.345 51.435) (end 93.345 49.595) (width 0.25) (layer B.Cu) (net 8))
 (segment (start 95.59 53.68) (end 103.89 53.68) (width 0.25) (layer F.Cu) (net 8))
 (segment (start 93.345 51.435) (end 95.59 53.68) (width 0.25) (layer F.Cu) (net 8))
 (segment (start 104.92 51.515) (end 104.755 51.68) (width 0.25) (layer F.Cu) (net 7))
 (segment (start 107.95 51.515) (end 104.92 51.515) (width 0.25) (layer F.Cu) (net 7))
 (segment (start 111.76 49.57) (end 109.26 49.57) (width 0.25) (layer F.Cu) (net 5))
 (segment (start 107.37 47.68) (end 104.755 47.68) (width 0.25) (layer F.Cu) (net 5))
 (segment (start 109.26 49.57) (end 107.37 47.68) (width 0.25) (layer F.Cu) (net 5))
 (via (at 95.885 51.435) (size 0.8) (drill 0.4) (layers F.Cu B.Cu) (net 2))
 (segment (start 110.584999 43.085001) (end 111.76 41.91) (width 0.25) (layer F.Cu) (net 2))
 (segment (start 108.655999 43.085001) (end 110.584999 43.085001) (width 0.25) (layer F.Cu) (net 2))
 (segment (start 107.250998 41.68) (end 108.655999 43.085001) (width 0.25) (layer F.Cu) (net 2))
 (segment (start 104.755 41.68) (end 107.250998 41.68) (width 0.25) (layer F.Cu) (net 2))
 (segment (start 95.885 49.595) (end 95.885 51.435) (width 0.25) (layer B.Cu) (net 2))
 (segment (start 95.885 51.435) (end 95.885 46.99) (width 0.25) (layer F.Cu) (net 2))
 (segment (start 101.195 41.68) (end 105.39 41.68) (width 0.25) (layer F.Cu) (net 2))
 (segment (start 95.885 46.99) (end 101.195 41.68) (width 0.25) (layer F.Cu) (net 2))
 (via (at 94.615 51.435) (size 0.8) (drill 0.4) (layers F.Cu B.Cu) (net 1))
 (segment (start 94.615 49.595) (end 94.615 51.435) (width 0.25) (layer B.Cu) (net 1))
 (segment (start 101.29 39.68) (end 105.39 39.68) (width 0.25) (layer F.Cu) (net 1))
 (segment (start 94.615 46.355) (end 101.29 39.68) (width 0.25) (layer F.Cu) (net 1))
 (segment (start 94.615 51.435) (end 94.615 46.355) (width 0.25) (layer F.Cu) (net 1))
 (segment (start 106.99 39.68) (end 109.22 41.91) (width 0.25) (layer F.Cu) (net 1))
 (segment (start 105.39 39.68) (end 106.99 39.68) (width 0.25) (layer F.Cu) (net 1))
 (segment (start 111.655 46.99) (end 111.735 47.07) (width 0.25) (layer F.Cu) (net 33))
 (segment (start 109.22 46.99) (end 111.655 46.99) (width 0.25) (layer F.Cu) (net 33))
 (segment (start 88.9475 39.68) (end 89.555 39.68) (width 0.25) (layer F.Cu) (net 16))
 (segment (start 89.415 39.68) (end 89.555 39.68) (width 0.25) (layer F.Cu) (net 16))
 (segment (start 86.36 36.625) (end 89.415 39.68) (width 0.25) (layer F.Cu) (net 16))
 (segment (start 76.2 36.83) (end 82.7 36.83) (width 0.25) (layer F.Cu) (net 16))
 (segment (start 86.155 36.83) (end 86.36 36.625) (width 0.25) (layer F.Cu) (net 16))
 (segment (start 82.7 36.83) (end 86.155 36.83) (width 0.25) (layer F.Cu) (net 16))
 (segment (start 88.3125 39.68) (end 89.555 39.68) (width 0.25) (layer F.Cu) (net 16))
 (segment (start 86.36 41.6325) (end 88.3125 39.68) (width 0.25) (layer F.Cu) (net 16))
 (segment (start 88.659999 48.784999) (end 89.555 49.68) (width 0.25) (layer F.Cu) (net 11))
 (segment (start 78.215001 48.784999) (end 88.659999 48.784999) (width 0.25) (layer F.Cu) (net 11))
 (segment (start 76.2 50.8) (end 78.215001 48.784999) (width 0.25) (layer F.Cu) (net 11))
 (segment (start 76.2 48.26) (end 76.2 48.411002) (width 0.25) (layer F.Cu) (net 12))
 (segment (start 76.78 47.68) (end 76.2 48.26) (width 0.25) (layer F.Cu) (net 12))
 (segment (start 89.61 48.26) (end 90.19 47.68) (width 0.25) (layer F.Cu) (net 12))
 (segment (start 76.2 48.26) (end 89.61 48.26) (width 0.25) (layer F.Cu) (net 12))
 (segment (start 86.654999 47.715001) (end 88.69 45.68) (width 0.25) (layer F.Cu) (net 13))
 (segment (start 88.69 45.68) (end 90.19 45.68) (width 0.25) (layer F.Cu) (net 13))
 (segment (start 78.195001 47.715001) (end 86.654999 47.715001) (width 0.25) (layer F.Cu) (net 13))
 (segment (start 76.2 45.72) (end 78.195001 47.715001) (width 0.25) (layer F.Cu) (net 13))
 (segment (start 107.64069 49.68) (end 104.755 49.68) (width 0.25) (layer F.Cu) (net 6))
 (segment (start 108.76069 50.8) (end 107.64069 49.68) (width 0.25) (layer F.Cu) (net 6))
 (segment (start 118.11 50.8) (end 108.76069 50.8) (width 0.25) (layer F.Cu) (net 6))
 (segment (start 108.835 48.26) (end 118.11 48.26) (width 0.25) (layer F.Cu) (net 4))
 (segment (start 106.255 45.68) (end 108.835 48.26) (width 0.25) (layer F.Cu) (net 4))
 (segment (start 104.755 45.68) (end 106.255 45.68) (width 0.25) (layer F.Cu) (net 4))
 (segment (start 105.090002 43.68) (end 104.755 43.68) (width 0.25) (layer F.Cu) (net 3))
 (segment (start 117.82749 45.43749) (end 118.11 45.72) (width 0.25) (layer F.Cu) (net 3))
 (segment (start 116.07 43.68) (end 118.11 45.72) (width 0.25) (layer F.Cu) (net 3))
 (segment (start 105.39 43.68) (end 116.07 43.68) (width 0.25) (layer F.Cu) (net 3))
 (via (at 79.375 46.99) (size 0.8) (drill 0.4) (layers F.Cu B.Cu) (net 10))
 (segment (start 79.86 50.11) (end 86.36 50.11) (width 0.25) (layer F.Cu) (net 10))
 (segment (start 87.93 51.68) (end 89.555 51.68) (width 0.25) (layer F.Cu) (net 10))
 (segment (start 86.36 50.11) (end 87.93 51.68) (width 0.25) (layer F.Cu) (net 10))
 (segment (start 79.86 47.475) (end 79.375 46.99) (width 0.25) (layer B.Cu) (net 10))
 (segment (start 79.86 50.11) (end 79.86 47.475) (width 0.25) (layer B.Cu) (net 10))
 (segment (start 79.375 45.8) (end 79.455 45.72) (width 0.25) (layer F.Cu) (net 10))
 (segment (start 79.375 46.99) (end 79.375 45.8) (width 0.25) (layer F.Cu) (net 10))
 (via (at 107.315 38.1) (size 0.8) (drill 0.4) (layers F.Cu B.Cu) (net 17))
 (segment (start 100.32 39.8) (end 100.09 40.03) (width 0.25) (layer B.Cu) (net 17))
 (segment (start 102.87 39.8) (end 100.32 39.8) (width 0.25) (layer B.Cu) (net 17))
 (segment (start 111.215 37.7) (end 111.215 36.777002) (width 0.25) (layer F.Cu) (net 17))
 (segment (start 111.215 36.777002) (end 113.067002 34.925) (width 0.25) (layer F.Cu) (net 17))
 (segment (start 116.115 36.939998) (end 116.115 37.7) (width 0.25) (layer F.Cu) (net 17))
 (segment (start 114.100002 34.925) (end 116.115 36.939998) (width 0.25) (layer F.Cu) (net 17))
 (segment (start 113.067002 34.925) (end 114.100002 34.925) (width 0.25) (layer F.Cu) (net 17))
 (segment (start 107.315 37.09826) (end 107.315 38.1) (width 0.25) (layer F.Cu) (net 17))
 (segment (start 109.48826 34.925) (end 107.315 37.09826) (width 0.25) (layer F.Cu) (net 17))
 (segment (start 113.067002 34.925) (end 109.48826 34.925) (width 0.25) (layer F.Cu) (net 17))
 (segment (start 105.615 39.8) (end 102.87 39.8) (width 0.25) (layer B.Cu) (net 17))
 (segment (start 107.315 38.1) (end 105.615 39.8) (width 0.25) (layer B.Cu) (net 17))
 (via (at 115.57 39.37) (size 0.8) (drill 0.4) (layers F.Cu B.Cu) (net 27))
 (segment (start 114.415 38.660002) (end 114.415 37.7) (width 0.25) (layer F.Cu) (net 27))
 (segment (start 114.325001 38.750001) (end 114.415 38.660002) (width 0.25) (layer F.Cu) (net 27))
 (segment (start 113.415 38.675) (end 113.490001 38.750001) (width 0.25) (layer F.Cu) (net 27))
 (segment (start 113.490001 38.750001) (end 114.325001 38.750001) (width 0.25) (layer F.Cu) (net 27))
 (segment (start 113.415 37.7) (end 113.415 38.675) (width 0.25) (layer F.Cu) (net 27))
 (segment (start 114.415 38.780685) (end 114.415 37.7) (width 0.25) (layer F.Cu) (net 27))
 (segment (start 115.004315 39.37) (end 114.415 38.780685) (width 0.25) (layer F.Cu) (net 27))
 (segment (start 115.57 39.37) (end 115.004315 39.37) (width 0.25) (layer F.Cu) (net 27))
 (segment (start 114.844999 40.095001) (end 115.57 39.37) (width 0.25) (layer B.Cu) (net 27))
 (segment (start 108.219999 40.095001) (end 114.844999 40.095001) (width 0.25) (layer B.Cu) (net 27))
 (segment (start 99.695 48.62) (end 108.219999 40.095001) (width 0.25) (layer B.Cu) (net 27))
 (segment (start 99.695 49.595) (end 99.695 48.62) (width 0.25) (layer B.Cu) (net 27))
 (via (at 110.49 39.37) (size 0.8) (drill 0.4) (layers F.Cu B.Cu) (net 28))
 (segment (start 113.915 36.725) (end 113.915 37.7) (width 0.25) (layer F.Cu) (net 28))
 (segment (start 113.004999 36.649999) (end 113.839999 36.649999) (width 0.25) (layer F.Cu) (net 28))
 (segment (start 113.839999 36.649999) (end 113.915 36.725) (width 0.25) (layer F.Cu) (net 28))
 (segment (start 112.915 36.739998) (end 113.004999 36.649999) (width 0.25) (layer F.Cu) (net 28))
 (segment (start 112.915 37.7) (end 112.915 36.739998) (width 0.25) (layer F.Cu) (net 28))
 (segment (start 112.915 38.675) (end 112.915 37.7) (width 0.25) (layer F.Cu) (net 28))
 (segment (start 112.22 39.37) (end 112.915 38.675) (width 0.25) (layer F.Cu) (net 28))
 (segment (start 110.49 39.37) (end 112.22 39.37) (width 0.25) (layer F.Cu) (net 28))
 (segment (start 108.273232 39.37) (end 98.425 49.218232) (width 0.25) (layer B.Cu) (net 28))
 (segment (start 98.425 49.218232) (end 98.425 49.595) (width 0.25) (layer B.Cu) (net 28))
 (segment (start 110.49 39.37) (end 108.273232 39.37) (width 0.25) (layer B.Cu) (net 28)))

